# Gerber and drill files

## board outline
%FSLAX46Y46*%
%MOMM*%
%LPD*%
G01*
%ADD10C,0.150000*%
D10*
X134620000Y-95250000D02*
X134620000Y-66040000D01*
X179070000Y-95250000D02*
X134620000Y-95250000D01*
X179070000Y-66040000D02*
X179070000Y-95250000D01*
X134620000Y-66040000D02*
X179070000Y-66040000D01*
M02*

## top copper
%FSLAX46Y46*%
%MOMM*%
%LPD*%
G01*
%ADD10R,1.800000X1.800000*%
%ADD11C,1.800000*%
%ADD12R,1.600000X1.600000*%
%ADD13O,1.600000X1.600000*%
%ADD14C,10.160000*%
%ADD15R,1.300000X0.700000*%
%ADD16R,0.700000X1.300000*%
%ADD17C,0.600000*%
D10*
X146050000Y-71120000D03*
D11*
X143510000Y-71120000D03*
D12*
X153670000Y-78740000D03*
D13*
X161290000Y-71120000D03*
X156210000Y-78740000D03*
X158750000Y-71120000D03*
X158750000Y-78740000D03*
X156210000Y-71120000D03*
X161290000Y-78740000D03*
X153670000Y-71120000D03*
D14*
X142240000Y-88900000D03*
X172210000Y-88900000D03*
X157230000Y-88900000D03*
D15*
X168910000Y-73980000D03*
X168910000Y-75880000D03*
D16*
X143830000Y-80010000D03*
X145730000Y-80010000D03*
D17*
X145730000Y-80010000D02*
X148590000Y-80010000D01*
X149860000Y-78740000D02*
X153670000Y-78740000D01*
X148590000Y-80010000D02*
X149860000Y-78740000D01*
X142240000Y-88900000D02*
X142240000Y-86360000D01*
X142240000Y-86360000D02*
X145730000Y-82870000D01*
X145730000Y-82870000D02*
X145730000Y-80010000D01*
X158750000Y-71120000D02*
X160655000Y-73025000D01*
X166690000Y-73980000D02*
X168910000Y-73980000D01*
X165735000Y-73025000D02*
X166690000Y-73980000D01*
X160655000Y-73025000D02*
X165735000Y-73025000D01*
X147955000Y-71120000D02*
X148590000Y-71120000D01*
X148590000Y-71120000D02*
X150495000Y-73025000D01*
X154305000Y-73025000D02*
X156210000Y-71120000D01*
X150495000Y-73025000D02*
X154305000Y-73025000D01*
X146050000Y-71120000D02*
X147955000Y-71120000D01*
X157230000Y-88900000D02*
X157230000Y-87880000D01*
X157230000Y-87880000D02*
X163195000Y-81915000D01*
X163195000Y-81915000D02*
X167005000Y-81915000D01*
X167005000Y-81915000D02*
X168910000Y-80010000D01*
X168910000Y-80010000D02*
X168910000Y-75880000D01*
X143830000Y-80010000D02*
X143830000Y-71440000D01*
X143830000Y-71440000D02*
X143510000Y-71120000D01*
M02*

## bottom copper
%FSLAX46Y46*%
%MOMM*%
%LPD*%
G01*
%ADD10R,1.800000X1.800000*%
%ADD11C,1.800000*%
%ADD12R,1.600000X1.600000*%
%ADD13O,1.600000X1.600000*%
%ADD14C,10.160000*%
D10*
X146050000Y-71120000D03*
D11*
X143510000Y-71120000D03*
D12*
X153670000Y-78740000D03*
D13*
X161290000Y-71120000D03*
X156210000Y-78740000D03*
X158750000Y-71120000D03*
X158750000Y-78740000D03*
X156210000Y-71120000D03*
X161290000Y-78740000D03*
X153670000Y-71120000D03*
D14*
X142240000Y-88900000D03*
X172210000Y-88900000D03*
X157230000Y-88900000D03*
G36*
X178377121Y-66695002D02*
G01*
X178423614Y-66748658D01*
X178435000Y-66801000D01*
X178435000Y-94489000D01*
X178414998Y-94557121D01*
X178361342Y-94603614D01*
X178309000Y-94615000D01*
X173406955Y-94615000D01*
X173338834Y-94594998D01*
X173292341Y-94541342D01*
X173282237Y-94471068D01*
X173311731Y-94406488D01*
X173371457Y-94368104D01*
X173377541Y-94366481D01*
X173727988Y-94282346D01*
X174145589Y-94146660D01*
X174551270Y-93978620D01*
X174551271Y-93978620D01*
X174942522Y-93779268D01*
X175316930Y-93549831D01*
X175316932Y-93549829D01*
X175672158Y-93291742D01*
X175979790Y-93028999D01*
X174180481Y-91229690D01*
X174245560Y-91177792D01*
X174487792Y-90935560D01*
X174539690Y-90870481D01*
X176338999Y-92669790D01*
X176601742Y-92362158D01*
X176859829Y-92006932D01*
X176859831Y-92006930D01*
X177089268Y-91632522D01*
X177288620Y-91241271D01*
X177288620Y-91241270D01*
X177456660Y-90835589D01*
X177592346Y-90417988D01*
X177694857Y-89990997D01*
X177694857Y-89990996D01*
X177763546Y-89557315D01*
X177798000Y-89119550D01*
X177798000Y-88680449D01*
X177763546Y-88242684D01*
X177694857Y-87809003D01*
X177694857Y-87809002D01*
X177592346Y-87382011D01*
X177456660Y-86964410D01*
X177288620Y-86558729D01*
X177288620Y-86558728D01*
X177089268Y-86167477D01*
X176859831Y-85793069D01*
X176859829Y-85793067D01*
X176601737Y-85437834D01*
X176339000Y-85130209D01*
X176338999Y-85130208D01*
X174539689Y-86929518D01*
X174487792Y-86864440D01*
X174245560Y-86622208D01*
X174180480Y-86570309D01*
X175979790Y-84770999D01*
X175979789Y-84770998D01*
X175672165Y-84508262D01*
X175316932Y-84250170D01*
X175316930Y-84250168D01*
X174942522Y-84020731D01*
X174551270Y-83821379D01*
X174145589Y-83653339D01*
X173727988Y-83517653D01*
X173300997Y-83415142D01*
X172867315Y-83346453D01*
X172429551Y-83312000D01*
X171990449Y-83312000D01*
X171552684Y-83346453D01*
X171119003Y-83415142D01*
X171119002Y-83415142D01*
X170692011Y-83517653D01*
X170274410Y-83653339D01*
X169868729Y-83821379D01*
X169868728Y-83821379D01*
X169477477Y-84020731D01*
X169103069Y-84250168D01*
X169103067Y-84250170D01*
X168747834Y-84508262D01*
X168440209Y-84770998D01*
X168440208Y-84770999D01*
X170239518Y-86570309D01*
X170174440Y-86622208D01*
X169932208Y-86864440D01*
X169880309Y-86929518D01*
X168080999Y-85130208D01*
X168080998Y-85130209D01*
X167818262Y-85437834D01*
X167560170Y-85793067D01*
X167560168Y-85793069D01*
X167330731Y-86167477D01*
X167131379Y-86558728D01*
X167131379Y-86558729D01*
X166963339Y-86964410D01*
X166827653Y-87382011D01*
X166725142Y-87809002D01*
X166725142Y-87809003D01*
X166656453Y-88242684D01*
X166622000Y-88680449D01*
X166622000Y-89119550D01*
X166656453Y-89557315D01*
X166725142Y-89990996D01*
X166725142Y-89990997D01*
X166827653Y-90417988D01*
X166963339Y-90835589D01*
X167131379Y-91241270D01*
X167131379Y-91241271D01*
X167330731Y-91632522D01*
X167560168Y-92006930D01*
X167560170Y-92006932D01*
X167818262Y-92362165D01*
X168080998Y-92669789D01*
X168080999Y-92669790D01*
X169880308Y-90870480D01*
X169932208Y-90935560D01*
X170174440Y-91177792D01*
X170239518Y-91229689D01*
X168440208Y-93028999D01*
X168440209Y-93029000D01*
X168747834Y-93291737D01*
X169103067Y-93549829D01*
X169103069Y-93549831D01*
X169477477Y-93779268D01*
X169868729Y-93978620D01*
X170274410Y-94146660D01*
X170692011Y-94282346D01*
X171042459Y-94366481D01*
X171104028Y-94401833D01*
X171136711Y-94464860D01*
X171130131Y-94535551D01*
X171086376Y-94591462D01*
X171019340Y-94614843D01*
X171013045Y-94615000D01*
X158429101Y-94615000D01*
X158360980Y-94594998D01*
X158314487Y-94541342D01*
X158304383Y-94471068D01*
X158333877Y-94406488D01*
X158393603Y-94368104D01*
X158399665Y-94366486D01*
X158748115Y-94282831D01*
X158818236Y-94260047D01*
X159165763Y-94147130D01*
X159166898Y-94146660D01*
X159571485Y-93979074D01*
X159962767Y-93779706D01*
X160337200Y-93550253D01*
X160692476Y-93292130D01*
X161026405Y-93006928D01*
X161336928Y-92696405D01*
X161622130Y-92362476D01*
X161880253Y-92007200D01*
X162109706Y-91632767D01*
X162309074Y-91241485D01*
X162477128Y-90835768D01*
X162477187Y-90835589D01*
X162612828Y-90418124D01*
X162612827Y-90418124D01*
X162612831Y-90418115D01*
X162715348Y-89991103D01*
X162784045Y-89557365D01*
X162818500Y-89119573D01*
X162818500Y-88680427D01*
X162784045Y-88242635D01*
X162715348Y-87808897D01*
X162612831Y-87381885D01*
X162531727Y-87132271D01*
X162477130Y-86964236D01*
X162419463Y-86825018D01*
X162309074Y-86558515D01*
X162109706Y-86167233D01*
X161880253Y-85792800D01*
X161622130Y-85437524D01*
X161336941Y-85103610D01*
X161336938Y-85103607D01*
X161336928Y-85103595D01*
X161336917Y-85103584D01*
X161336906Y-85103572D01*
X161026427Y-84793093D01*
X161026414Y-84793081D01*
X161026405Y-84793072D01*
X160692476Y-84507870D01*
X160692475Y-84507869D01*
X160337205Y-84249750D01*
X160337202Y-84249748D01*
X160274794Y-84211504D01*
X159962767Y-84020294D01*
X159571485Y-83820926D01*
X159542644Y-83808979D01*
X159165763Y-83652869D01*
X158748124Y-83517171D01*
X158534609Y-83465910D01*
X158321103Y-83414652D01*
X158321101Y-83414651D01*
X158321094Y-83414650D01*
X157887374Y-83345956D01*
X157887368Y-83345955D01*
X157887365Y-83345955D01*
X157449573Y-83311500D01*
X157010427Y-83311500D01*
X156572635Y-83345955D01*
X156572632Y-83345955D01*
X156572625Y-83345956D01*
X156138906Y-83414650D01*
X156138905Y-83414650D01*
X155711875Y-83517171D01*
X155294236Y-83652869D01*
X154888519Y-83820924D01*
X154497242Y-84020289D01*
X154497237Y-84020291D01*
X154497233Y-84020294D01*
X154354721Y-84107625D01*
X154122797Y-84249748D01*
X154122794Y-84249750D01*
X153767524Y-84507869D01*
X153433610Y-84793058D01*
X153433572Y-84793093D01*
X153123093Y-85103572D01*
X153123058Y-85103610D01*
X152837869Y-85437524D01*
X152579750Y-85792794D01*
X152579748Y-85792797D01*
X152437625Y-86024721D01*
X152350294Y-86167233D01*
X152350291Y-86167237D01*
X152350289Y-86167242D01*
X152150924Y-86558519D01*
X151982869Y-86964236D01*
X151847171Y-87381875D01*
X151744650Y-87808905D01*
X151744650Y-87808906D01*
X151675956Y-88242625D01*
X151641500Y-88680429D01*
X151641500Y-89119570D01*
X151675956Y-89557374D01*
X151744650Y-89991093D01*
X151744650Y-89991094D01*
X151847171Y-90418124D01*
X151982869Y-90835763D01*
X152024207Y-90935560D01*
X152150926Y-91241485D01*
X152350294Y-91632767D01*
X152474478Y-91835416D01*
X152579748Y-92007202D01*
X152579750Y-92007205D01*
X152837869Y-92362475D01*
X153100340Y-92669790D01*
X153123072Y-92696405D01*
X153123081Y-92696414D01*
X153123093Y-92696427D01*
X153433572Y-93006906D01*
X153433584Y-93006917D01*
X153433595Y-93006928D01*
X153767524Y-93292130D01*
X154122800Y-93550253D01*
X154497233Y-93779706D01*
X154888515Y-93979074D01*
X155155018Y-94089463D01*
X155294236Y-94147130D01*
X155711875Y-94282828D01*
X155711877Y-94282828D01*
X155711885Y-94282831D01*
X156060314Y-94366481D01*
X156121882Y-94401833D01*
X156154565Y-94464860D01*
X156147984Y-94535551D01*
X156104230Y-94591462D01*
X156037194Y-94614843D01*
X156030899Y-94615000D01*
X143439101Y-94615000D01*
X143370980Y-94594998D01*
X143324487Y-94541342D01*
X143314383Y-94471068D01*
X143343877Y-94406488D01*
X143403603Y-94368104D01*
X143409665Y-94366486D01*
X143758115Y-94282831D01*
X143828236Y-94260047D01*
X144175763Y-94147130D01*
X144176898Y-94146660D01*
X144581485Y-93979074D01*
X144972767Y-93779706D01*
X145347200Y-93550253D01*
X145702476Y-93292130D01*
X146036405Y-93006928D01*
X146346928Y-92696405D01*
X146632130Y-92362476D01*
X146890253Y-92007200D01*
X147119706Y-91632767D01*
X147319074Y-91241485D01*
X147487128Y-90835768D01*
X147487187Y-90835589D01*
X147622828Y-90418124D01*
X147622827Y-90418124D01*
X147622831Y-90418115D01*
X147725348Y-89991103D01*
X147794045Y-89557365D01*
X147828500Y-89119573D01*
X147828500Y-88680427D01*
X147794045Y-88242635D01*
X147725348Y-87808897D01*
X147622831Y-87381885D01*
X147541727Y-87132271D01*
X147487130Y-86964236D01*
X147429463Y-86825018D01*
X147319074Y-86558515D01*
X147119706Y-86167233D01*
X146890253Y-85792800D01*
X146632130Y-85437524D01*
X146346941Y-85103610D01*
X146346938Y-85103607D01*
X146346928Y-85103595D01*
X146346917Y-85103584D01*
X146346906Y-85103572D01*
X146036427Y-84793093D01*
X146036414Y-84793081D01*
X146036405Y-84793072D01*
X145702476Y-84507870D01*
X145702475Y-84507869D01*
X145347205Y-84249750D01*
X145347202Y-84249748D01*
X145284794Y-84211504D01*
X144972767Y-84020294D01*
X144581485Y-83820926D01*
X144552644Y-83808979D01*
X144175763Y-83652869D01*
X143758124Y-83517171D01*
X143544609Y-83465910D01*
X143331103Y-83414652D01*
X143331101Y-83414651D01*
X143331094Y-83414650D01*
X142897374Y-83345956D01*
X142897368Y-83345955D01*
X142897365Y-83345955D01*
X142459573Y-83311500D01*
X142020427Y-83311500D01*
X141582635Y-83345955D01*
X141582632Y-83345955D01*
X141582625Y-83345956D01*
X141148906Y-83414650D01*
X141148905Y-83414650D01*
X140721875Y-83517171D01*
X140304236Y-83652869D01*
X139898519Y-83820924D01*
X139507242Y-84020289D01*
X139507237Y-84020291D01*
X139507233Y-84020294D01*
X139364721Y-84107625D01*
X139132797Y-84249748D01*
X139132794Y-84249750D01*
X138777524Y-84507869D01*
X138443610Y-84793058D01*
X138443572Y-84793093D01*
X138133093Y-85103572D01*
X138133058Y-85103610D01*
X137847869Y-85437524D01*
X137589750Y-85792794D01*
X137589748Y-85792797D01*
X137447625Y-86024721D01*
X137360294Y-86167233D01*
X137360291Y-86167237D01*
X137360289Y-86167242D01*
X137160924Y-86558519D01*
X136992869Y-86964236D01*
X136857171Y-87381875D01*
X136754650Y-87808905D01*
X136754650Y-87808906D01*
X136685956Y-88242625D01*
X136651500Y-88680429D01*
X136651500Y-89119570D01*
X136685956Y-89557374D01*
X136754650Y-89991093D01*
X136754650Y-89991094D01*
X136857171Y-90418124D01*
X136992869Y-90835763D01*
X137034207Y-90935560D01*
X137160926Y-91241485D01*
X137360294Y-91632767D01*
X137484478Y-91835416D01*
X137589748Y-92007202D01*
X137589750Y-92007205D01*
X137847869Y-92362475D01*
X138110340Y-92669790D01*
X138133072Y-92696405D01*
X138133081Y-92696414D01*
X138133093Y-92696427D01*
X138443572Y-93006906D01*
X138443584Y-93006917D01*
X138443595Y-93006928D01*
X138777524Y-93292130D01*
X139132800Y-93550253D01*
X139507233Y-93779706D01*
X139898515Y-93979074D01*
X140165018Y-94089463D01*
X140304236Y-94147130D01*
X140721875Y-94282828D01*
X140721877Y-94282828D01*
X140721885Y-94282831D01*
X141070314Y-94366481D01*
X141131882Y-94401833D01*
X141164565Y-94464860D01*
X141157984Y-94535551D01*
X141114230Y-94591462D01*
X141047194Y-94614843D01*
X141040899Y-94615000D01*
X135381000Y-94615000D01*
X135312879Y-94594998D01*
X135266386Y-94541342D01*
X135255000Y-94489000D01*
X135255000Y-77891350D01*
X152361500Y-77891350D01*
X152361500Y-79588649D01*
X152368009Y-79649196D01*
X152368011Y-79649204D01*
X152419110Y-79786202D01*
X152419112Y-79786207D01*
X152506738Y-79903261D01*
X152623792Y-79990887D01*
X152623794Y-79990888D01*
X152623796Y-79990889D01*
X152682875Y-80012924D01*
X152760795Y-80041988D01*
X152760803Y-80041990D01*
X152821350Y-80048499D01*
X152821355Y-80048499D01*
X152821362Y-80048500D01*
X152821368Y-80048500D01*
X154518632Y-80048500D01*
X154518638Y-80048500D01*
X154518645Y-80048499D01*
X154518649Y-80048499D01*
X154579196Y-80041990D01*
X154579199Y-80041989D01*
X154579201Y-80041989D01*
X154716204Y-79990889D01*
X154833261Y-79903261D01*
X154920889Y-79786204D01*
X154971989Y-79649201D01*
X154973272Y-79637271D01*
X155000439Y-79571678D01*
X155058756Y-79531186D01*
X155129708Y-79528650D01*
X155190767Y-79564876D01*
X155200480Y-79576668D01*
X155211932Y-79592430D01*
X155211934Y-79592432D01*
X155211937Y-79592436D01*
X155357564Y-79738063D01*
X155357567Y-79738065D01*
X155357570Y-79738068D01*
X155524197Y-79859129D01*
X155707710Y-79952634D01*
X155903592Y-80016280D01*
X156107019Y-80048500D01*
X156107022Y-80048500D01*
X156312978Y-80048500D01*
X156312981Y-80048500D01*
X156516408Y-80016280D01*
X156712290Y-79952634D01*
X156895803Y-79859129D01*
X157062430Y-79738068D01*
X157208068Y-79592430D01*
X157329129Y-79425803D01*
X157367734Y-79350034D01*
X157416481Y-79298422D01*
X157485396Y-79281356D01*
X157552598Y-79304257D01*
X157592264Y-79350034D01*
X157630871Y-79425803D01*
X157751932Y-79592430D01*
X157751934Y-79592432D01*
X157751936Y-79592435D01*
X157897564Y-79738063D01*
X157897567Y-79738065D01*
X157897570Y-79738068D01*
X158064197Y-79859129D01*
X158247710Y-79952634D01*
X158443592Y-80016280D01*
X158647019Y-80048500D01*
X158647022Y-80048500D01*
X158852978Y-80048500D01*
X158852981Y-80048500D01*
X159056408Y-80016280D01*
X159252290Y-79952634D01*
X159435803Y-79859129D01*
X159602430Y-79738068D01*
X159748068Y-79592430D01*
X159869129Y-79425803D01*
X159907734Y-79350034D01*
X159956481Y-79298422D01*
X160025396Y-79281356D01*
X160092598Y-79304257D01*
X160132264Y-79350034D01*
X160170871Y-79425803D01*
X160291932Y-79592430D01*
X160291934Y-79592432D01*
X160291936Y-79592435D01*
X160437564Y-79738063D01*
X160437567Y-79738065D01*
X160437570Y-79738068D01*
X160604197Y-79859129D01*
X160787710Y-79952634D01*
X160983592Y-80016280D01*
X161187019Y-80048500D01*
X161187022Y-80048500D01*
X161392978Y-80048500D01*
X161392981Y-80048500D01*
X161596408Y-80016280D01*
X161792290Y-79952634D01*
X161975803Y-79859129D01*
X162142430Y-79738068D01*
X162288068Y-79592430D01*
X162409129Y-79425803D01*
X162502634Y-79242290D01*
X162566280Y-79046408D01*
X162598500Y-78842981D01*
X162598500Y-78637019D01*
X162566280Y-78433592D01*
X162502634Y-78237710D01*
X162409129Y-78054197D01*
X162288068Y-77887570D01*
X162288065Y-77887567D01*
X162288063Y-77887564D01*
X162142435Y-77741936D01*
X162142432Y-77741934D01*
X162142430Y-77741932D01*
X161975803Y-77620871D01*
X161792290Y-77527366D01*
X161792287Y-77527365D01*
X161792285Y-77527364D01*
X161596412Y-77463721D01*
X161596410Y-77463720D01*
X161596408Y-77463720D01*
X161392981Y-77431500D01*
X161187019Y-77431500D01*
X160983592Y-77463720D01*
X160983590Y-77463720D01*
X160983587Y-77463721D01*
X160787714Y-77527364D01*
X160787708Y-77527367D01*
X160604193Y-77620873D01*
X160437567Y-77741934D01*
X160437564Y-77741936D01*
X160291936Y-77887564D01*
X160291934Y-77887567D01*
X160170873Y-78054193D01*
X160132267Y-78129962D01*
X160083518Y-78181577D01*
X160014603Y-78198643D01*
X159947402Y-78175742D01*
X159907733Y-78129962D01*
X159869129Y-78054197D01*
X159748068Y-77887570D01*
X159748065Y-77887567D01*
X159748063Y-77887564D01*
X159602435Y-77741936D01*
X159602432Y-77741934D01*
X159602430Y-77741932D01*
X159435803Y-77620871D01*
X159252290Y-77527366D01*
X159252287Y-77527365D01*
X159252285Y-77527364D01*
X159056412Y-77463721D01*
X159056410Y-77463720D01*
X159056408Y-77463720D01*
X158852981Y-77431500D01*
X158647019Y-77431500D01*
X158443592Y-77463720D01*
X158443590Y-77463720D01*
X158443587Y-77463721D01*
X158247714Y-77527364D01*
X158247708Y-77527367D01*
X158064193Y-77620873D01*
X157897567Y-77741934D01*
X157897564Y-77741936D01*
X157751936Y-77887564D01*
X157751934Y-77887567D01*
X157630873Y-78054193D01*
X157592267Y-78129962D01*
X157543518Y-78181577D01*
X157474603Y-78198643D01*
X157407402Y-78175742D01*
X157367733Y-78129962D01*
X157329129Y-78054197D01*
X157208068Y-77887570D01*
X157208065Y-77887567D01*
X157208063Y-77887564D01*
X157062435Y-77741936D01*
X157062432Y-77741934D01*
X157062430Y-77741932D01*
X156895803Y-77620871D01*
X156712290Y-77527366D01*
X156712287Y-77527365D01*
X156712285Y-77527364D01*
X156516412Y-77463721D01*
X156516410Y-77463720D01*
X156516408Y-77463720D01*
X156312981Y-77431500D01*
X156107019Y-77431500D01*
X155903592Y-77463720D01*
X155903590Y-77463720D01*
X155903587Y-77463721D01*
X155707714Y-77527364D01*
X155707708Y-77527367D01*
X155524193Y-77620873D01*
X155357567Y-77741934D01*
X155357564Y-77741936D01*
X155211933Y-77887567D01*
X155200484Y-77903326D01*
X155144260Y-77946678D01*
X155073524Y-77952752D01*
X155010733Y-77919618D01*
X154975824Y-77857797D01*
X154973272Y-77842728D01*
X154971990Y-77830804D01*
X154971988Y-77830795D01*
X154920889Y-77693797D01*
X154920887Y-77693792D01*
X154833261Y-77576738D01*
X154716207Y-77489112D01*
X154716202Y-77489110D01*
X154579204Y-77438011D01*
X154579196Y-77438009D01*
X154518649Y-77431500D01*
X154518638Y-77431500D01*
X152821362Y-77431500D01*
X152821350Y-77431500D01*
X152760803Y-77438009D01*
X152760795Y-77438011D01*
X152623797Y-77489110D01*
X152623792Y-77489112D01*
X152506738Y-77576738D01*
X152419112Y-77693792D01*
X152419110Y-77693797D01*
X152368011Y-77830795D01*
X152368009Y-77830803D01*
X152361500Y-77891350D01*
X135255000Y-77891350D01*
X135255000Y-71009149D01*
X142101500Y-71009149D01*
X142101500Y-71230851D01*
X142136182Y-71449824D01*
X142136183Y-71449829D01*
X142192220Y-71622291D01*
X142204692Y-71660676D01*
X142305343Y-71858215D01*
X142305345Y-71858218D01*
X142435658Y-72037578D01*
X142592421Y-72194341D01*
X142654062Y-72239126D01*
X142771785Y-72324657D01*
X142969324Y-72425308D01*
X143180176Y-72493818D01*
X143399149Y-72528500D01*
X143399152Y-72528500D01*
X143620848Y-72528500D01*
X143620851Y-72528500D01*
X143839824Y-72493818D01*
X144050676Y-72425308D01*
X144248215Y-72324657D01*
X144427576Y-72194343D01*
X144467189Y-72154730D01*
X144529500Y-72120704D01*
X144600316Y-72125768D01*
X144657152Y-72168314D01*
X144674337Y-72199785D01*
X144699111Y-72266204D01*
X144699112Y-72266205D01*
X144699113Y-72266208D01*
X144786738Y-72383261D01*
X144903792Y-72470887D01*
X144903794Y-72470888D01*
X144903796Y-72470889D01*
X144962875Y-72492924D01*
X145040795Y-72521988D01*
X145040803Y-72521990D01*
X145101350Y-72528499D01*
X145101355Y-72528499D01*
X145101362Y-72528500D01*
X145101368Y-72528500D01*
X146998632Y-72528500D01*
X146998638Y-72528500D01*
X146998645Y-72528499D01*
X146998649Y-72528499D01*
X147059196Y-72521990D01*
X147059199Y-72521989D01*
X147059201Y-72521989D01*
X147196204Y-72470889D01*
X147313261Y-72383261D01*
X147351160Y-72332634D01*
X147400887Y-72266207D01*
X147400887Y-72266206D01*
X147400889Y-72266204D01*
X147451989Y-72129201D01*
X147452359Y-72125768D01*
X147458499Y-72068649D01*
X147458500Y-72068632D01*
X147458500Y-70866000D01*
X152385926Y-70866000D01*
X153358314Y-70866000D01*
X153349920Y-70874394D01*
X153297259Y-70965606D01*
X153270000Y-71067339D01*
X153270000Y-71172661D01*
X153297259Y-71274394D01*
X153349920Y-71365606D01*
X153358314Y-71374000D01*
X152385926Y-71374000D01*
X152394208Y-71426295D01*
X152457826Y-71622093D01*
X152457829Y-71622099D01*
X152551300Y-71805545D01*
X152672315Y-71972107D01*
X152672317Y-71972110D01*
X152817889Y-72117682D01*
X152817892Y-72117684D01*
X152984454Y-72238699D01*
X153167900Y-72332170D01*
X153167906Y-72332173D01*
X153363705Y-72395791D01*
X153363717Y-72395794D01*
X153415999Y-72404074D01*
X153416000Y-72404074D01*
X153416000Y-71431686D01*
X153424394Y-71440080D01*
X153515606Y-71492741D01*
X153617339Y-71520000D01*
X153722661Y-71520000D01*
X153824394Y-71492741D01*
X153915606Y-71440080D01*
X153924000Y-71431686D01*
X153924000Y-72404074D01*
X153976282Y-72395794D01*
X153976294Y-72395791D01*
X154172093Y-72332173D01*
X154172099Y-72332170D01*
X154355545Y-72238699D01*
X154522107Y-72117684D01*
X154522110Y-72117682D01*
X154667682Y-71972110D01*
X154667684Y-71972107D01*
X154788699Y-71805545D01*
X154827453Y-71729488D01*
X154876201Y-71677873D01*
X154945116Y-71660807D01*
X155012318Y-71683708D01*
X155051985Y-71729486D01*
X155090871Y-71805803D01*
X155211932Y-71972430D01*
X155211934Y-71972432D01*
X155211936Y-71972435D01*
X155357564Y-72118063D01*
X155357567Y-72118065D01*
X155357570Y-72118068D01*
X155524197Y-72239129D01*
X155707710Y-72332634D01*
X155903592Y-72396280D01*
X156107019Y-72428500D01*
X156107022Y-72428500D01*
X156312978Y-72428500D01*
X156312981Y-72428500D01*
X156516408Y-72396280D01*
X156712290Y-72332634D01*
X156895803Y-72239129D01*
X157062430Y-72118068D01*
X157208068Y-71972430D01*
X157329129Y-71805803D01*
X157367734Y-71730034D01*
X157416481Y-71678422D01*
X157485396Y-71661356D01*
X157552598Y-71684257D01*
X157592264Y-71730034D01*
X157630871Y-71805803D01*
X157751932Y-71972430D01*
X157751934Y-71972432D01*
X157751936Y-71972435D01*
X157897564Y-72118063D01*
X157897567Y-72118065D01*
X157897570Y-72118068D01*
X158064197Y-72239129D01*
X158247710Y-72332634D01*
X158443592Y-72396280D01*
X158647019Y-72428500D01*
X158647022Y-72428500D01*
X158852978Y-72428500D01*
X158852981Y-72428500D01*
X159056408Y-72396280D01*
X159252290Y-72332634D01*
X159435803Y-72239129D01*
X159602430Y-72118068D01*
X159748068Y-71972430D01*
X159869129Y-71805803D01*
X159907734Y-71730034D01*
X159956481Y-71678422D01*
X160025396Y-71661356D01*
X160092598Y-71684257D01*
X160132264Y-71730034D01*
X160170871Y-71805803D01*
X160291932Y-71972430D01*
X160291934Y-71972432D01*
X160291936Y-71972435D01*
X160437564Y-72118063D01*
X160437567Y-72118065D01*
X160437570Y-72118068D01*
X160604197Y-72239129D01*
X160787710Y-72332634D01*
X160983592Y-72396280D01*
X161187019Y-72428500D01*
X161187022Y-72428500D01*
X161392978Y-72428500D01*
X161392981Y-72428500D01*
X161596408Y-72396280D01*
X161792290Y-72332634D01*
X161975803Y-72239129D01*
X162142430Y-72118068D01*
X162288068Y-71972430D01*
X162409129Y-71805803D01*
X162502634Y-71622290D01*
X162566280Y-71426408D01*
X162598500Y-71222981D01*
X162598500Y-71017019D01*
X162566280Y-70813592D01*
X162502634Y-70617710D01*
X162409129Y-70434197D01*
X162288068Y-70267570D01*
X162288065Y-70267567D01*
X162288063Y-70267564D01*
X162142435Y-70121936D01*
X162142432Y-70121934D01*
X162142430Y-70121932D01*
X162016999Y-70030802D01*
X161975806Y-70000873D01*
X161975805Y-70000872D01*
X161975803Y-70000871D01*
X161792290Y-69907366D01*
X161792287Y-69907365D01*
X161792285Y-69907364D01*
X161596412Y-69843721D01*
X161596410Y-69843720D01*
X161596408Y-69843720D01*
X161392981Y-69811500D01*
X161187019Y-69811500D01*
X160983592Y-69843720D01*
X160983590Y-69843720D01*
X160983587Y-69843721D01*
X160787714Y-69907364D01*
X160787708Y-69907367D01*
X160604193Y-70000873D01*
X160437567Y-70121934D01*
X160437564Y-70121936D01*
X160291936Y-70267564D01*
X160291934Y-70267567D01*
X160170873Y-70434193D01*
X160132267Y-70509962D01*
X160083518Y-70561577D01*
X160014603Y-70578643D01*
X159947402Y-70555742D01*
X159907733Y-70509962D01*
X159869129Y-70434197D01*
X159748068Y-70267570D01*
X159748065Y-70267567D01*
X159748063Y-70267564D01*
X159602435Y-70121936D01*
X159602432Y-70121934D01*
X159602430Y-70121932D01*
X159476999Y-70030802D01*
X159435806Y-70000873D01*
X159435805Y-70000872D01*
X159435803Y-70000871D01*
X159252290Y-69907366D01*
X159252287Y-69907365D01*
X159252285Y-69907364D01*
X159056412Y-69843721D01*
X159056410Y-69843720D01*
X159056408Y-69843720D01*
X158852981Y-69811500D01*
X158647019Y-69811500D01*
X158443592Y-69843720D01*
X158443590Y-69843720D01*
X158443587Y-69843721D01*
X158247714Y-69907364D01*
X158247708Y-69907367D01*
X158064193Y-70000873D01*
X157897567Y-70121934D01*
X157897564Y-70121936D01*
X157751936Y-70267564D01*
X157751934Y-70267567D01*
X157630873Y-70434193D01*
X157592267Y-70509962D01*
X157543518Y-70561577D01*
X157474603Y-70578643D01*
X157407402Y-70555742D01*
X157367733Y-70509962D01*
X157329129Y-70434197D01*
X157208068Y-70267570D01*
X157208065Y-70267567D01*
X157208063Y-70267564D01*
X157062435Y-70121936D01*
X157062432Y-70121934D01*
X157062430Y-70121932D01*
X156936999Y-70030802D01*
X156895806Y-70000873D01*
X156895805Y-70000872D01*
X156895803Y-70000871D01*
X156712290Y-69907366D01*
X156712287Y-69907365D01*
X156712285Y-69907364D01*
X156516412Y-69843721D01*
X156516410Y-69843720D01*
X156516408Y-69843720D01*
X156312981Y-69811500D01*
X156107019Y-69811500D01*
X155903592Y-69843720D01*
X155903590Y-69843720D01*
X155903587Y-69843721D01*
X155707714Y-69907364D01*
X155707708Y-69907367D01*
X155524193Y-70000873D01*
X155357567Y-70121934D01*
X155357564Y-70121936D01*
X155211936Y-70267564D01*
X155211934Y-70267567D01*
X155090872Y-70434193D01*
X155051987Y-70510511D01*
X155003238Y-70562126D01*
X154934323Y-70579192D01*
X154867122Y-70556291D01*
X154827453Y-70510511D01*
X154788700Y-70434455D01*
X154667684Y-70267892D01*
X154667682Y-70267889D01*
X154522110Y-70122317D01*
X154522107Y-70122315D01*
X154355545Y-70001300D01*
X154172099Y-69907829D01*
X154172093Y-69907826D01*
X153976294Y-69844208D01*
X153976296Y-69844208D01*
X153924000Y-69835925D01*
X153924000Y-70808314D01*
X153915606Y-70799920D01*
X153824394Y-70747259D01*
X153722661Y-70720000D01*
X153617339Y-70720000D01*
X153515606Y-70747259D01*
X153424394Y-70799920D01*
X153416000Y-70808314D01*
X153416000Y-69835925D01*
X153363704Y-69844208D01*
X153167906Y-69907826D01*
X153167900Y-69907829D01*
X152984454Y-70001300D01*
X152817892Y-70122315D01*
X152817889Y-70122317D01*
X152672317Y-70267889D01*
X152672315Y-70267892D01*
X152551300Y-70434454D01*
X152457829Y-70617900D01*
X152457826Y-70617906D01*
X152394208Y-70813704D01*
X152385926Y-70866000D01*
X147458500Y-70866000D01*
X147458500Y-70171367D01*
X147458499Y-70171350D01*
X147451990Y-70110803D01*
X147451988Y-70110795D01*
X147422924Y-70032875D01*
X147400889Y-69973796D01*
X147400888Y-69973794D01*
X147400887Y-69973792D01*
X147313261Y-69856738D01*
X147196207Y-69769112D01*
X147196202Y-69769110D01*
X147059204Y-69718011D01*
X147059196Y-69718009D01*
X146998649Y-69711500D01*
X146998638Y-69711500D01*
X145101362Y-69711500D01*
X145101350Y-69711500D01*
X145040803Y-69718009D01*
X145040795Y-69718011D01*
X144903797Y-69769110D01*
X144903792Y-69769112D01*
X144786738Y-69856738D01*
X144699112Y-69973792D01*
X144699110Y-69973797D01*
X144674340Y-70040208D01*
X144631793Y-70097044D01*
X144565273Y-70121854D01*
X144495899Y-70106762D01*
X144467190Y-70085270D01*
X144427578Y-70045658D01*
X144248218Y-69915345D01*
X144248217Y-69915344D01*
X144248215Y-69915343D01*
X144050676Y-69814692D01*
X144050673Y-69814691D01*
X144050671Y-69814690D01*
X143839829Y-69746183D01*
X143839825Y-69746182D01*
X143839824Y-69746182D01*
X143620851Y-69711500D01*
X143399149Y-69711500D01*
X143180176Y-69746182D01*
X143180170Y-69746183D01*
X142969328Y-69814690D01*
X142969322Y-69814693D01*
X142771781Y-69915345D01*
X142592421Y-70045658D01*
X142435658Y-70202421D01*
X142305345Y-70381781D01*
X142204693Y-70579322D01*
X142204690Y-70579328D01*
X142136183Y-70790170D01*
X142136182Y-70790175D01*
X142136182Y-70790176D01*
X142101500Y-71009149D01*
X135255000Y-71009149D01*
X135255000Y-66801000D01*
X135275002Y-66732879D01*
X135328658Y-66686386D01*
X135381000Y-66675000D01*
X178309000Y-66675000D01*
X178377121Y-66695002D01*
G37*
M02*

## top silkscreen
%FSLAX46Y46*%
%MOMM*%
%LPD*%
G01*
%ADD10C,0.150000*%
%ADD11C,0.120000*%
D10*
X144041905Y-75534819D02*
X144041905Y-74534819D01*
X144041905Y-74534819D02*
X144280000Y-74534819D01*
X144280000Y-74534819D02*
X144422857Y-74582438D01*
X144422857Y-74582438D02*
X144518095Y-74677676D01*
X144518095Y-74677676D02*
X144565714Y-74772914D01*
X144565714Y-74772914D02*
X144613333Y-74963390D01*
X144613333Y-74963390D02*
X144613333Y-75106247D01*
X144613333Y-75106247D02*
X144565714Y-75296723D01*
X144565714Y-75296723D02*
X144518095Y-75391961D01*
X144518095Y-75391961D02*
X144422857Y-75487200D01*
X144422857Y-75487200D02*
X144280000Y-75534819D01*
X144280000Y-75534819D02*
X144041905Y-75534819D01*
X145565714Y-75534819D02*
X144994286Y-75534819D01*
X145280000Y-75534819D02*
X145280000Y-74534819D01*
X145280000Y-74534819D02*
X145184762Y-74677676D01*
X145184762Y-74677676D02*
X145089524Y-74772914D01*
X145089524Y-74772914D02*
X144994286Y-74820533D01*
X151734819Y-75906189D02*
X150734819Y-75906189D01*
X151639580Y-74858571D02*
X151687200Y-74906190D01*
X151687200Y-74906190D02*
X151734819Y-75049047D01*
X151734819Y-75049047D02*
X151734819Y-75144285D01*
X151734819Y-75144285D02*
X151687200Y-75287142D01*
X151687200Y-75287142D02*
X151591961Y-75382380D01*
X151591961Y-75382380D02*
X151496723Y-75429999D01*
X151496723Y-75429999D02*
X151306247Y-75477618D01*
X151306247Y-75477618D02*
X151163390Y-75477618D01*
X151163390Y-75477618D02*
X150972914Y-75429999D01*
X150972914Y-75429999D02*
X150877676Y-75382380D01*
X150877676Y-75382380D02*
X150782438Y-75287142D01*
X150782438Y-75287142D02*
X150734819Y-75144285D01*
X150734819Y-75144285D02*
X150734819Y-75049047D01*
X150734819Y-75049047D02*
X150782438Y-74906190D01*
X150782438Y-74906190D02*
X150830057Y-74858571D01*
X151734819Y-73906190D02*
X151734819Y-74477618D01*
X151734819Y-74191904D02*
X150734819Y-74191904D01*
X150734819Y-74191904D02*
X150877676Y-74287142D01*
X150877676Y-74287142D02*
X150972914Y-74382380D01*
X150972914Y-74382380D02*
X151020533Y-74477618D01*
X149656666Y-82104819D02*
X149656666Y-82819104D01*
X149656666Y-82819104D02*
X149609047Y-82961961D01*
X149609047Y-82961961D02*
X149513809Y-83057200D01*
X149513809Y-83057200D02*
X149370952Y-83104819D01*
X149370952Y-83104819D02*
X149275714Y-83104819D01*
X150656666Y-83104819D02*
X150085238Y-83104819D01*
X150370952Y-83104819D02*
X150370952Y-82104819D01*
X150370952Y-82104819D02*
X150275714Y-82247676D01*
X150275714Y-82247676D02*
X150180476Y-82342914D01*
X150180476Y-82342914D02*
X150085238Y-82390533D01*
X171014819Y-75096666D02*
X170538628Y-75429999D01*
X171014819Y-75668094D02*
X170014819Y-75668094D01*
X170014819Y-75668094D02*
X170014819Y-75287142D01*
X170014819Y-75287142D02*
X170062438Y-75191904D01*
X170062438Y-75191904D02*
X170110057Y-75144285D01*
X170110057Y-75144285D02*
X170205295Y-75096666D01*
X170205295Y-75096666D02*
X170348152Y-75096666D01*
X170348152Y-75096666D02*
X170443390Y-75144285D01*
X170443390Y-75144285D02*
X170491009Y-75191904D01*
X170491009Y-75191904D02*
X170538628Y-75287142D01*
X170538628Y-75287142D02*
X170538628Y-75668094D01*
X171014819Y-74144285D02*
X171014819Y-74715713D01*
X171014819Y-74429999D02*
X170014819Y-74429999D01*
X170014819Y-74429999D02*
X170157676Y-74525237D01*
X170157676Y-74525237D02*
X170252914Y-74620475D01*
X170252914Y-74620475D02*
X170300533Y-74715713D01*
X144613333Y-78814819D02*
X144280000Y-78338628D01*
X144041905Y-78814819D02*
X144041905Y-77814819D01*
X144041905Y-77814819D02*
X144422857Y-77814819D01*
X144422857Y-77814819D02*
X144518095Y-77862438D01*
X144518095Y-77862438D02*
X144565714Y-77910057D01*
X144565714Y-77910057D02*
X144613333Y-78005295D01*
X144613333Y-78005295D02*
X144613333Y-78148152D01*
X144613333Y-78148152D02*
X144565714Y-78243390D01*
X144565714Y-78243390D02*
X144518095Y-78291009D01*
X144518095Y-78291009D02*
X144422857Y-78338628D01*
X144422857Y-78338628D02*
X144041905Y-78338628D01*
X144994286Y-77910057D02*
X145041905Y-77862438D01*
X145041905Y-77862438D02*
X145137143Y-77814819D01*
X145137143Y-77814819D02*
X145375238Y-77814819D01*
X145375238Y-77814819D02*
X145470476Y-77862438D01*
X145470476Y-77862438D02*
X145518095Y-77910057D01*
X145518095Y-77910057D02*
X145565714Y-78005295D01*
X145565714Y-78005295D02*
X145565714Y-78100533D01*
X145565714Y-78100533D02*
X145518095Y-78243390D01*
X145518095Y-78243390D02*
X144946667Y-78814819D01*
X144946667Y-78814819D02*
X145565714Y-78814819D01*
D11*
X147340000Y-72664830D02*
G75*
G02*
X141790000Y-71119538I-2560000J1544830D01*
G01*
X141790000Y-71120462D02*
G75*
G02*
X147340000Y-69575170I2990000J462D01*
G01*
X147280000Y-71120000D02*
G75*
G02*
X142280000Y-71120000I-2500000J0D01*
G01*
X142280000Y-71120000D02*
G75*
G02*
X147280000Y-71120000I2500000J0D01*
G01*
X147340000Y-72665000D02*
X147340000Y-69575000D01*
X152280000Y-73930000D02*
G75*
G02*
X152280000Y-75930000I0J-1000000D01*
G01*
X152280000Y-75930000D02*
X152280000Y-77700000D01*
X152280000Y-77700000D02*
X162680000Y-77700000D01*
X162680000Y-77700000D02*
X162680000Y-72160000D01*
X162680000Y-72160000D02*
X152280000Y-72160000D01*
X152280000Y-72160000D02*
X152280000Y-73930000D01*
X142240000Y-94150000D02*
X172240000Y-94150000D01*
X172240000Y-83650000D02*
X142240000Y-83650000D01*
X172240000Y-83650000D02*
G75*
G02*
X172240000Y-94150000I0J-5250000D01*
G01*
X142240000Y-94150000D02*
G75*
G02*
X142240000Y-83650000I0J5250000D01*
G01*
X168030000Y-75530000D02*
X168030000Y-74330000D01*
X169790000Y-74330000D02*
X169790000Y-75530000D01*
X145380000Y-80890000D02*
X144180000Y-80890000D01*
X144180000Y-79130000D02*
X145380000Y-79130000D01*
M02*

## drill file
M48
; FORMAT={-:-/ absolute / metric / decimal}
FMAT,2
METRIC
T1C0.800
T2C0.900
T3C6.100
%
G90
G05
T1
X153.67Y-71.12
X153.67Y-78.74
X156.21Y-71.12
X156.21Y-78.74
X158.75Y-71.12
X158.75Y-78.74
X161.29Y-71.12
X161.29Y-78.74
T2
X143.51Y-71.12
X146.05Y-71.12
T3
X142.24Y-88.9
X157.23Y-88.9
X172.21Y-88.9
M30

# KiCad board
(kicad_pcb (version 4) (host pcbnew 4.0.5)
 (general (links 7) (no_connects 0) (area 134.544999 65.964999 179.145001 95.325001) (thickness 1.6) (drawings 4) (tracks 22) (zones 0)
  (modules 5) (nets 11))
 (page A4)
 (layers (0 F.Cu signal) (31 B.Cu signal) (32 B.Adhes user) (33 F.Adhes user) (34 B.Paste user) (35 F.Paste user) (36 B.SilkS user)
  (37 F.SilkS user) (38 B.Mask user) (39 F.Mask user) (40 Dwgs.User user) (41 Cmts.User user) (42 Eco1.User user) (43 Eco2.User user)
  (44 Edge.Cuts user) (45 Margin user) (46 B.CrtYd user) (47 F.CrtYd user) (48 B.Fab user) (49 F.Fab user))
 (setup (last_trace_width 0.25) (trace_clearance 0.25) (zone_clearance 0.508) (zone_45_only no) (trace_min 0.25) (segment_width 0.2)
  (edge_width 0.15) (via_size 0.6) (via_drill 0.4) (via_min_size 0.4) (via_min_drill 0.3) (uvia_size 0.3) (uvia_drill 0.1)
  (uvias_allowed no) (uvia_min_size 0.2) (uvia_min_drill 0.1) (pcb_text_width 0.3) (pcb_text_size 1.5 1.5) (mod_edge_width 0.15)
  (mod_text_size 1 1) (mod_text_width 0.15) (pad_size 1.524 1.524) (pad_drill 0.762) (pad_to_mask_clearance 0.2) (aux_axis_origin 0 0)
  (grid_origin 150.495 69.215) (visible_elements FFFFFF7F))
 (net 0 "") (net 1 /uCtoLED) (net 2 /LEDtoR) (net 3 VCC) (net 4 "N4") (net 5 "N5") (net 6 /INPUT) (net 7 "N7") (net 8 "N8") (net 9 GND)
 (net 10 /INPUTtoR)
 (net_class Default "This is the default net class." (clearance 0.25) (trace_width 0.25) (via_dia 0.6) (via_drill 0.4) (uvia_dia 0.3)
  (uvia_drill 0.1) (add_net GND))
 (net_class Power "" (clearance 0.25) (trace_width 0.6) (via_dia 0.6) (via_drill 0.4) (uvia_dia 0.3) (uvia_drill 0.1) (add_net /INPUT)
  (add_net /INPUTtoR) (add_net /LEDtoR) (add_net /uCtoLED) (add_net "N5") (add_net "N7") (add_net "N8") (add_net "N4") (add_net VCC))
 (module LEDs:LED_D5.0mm (layer F.Cu) (at 146.05 71.12 180)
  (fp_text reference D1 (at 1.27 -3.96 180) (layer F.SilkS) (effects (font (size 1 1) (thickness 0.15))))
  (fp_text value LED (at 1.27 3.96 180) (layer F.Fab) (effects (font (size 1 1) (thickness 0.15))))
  (fp_arc (start 1.27 0) (end -1.29 -1.54483) (angle 148.9) (layer F.SilkS) (width 0.12))
  (fp_arc (start 1.27 0) (end -1.29 1.54483) (angle -148.9) (layer F.SilkS) (width 0.12))
  (fp_circle (center 1.27 0) (end 3.77 0) (layer F.SilkS) (width 0.12))
  (fp_line (start -1.29 -1.545) (end -1.29 1.545) (layer F.SilkS) (width 0.12))
  (pad 1 thru_hole rect (at 0 0 180) (size 1.8 1.8) (drill 0.9) (layers *.Cu *.Mask) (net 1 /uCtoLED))
  (pad 2 thru_hole circle (at 2.54 0 180) (size 1.8 1.8) (drill 0.9) (layers *.Cu *.Mask) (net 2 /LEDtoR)))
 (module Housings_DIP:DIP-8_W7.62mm (layer F.Cu) (at 153.67 78.74 90)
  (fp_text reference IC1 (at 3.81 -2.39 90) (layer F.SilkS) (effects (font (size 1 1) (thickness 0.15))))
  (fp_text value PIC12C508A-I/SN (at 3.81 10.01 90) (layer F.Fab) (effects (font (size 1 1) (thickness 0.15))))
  (fp_arc (start 3.81 -1.39) (end 2.81 -1.39) (angle -180) (layer F.SilkS) (width 0.12))
  (fp_line (start 2.81 -1.39) (end 1.04 -1.39) (layer F.SilkS) (width 0.12))
  (fp_line (start 1.04 -1.39) (end 1.04 9.01) (layer F.SilkS) (width 0.12))
  (fp_line (start 1.04 9.01) (end 6.58 9.01) (layer F.SilkS) (width 0.12))
  (fp_line (start 6.58 9.01) (end 6.58 -1.39) (layer F.SilkS) (width 0.12))
  (fp_line (start 6.58 -1.39) (end 4.81 -1.39) (layer F.SilkS) (width 0.12))
  (pad 1 thru_hole rect (at 0 0 90) (size 1.6 1.6) (drill 0.8) (layers *.Cu *.Mask) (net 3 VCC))
  (pad 5 thru_hole oval (at 7.62 7.62 90) (size 1.6 1.6) (drill 0.8) (layers *.Cu *.Mask) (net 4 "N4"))
  (pad 2 thru_hole oval (at 0 2.54 90) (size 1.6 1.6) (drill 0.8) (layers *.Cu *.Mask) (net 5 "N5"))
  (pad 6 thru_hole oval (at 7.62 5.08 90) (size 1.6 1.6) (drill 0.8) (layers *.Cu *.Mask) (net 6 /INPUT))
  (pad 3 thru_hole oval (at 0 5.08 90) (size 1.6 1.6) (drill 0.8) (layers *.Cu *.Mask) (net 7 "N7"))
  (pad 7 thru_hole oval (at 7.62 2.54 90) (size 1.6 1.6) (drill 0.8) (layers *.Cu *.Mask) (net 1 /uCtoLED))
  (pad 4 thru_hole oval (at 0 7.62 90) (size 1.6 1.6) (drill 0.8) (layers *.Cu *.Mask) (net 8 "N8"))
  (pad 8 thru_hole oval (at 7.62 0 90) (size 1.6 1.6) (drill 0.8) (layers *.Cu *.Mask) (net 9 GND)))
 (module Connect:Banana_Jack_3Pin (layer F.Cu) (at 142.24 88.9)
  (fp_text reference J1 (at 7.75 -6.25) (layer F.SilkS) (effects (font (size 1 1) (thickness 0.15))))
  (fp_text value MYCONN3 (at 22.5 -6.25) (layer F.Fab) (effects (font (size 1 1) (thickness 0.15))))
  (fp_line (start 0 5.25) (end 30 5.25) (layer F.SilkS) (width 0.12))
  (fp_line (start 30 -5.25) (end 0 -5.25) (layer F.SilkS) (width 0.12))
  (fp_arc (start 30 0) (end 30 -5.25) (angle 180) (layer F.SilkS) (width 0.12))
  (fp_arc (start 0 0) (end 0 5.25) (angle 180) (layer F.SilkS) (width 0.12))
  (pad 1 thru_hole circle (at 0 0) (size 10.16 10.16) (drill 6.1) (layers *.Cu *.Mask) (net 3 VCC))
  (pad 3 thru_hole circle (at 29.97 0) (size 10.16 10.16) (drill 6.1) (layers *.Cu *.Mask) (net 9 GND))
  (pad 2 thru_hole circle (at 14.99 0) (size 10.16 10.16) (drill 6.1) (layers *.Cu *.Mask) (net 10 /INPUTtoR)))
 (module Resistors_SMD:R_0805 (layer F.Cu) (at 168.91 74.93 270)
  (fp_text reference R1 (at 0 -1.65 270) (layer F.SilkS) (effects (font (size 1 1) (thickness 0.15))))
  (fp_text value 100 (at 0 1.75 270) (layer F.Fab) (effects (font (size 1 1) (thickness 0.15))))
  (fp_line (start 0.6 0.88) (end -0.6 0.88) (layer F.SilkS) (width 0.12))
  (fp_line (start -0.6 -0.88) (end 0.6 -0.88) (layer F.SilkS) (width 0.12))
  (pad 1 smd rect (at -0.95 0 270) (size 0.7 1.3) (layers F.Cu F.Paste F.Mask) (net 6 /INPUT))
  (pad 2 smd rect (at 0.95 0 270) (size 0.7 1.3) (layers F.Cu F.Paste F.Mask) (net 10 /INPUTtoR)))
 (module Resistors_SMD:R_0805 (layer F.Cu) (at 144.78 80.01)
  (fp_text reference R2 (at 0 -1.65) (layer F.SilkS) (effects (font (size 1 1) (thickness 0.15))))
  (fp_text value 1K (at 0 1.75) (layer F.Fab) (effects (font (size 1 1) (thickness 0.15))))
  (fp_line (start 0.6 0.88) (end -0.6 0.88) (layer F.SilkS) (width 0.12))
  (fp_line (start -0.6 -0.88) (end 0.6 -0.88) (layer F.SilkS) (width 0.12))
  (pad 1 smd rect (at -0.95 0) (size 0.7 1.3) (layers F.Cu F.Paste F.Mask) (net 2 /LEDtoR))
  (pad 2 smd rect (at 0.95 0) (size 0.7 1.3) (layers F.Cu F.Paste F.Mask) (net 3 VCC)))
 (gr_line (start 134.62 95.25) (end 134.62 66.04) (angle 90) (layer Edge.Cuts) (width 0.15))
 (gr_line (start 179.07 95.25) (end 134.62 95.25) (angle 90) (layer Edge.Cuts) (width 0.15))
 (gr_line (start 179.07 66.04) (end 179.07 95.25) (angle 90) (layer Edge.Cuts) (width 0.15))
 (gr_line (start 134.62 66.04) (end 179.07 66.04) (angle 90) (layer Edge.Cuts) (width 0.15))
 (segment (start 145.73 80.01) (end 148.59 80.01) (width 0.6) (layer F.Cu) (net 3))
 (segment (start 149.86 78.74) (end 153.67 78.74) (width 0.6) (layer F.Cu) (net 3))
 (segment (start 148.59 80.01) (end 149.86 78.74) (width 0.6) (layer F.Cu) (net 3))
 (segment (start 142.24 88.9) (end 142.24 86.36) (width 0.6) (layer F.Cu) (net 3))
 (segment (start 142.24 86.36) (end 145.73 82.87) (width 0.6) (layer F.Cu) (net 3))
 (segment (start 145.73 82.87) (end 145.73 80.01) (width 0.6) (layer F.Cu) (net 3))
 (segment (start 158.75 71.12) (end 160.655 73.025) (width 0.6) (layer F.Cu) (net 6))
 (segment (start 166.69 73.98) (end 168.91 73.98) (width 0.6) (layer F.Cu) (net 6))
 (segment (start 165.735 73.025) (end 166.69 73.98) (width 0.6) (layer F.Cu) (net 6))
 (segment (start 160.655 73.025) (end 165.735 73.025) (width 0.6) (layer F.Cu) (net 6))
 (segment (start 147.955 71.12) (end 148.59 71.12) (width 0.6) (layer F.Cu) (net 1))
 (segment (start 148.59 71.12) (end 150.495 73.025) (width 0.6) (layer F.Cu) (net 1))
 (segment (start 154.305 73.025) (end 156.21 71.12) (width 0.6) (layer F.Cu) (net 1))
 (segment (start 150.495 73.025) (end 154.305 73.025) (width 0.6) (layer F.Cu) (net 1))
 (segment (start 146.05 71.12) (end 147.955 71.12) (width 0.6) (layer F.Cu) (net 1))
 (segment (start 157.23 88.9) (end 157.23 87.88) (width 0.6) (layer F.Cu) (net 10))
 (segment (start 157.23 87.88) (end 163.195 81.915) (width 0.6) (layer F.Cu) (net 10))
 (segment (start 163.195 81.915) (end 167.005 81.915) (width 0.6) (layer F.Cu) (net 10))
 (segment (start 167.005 81.915) (end 168.91 80.01) (width 0.6) (layer F.Cu) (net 10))
 (segment (start 168.91 80.01) (end 168.91 75.88) (width 0.6) (layer F.Cu) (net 10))
 (segment (start 143.83 80.01) (end 143.83 71.44) (width 0.6) (layer F.Cu) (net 2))
 (segment (start 143.83 71.44) (end 143.51 71.12) (width 0.6) (layer F.Cu) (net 2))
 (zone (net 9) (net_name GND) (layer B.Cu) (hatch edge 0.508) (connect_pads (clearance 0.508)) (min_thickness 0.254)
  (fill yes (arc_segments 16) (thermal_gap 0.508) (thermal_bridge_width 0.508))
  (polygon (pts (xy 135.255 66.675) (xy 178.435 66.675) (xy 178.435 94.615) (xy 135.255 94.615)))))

